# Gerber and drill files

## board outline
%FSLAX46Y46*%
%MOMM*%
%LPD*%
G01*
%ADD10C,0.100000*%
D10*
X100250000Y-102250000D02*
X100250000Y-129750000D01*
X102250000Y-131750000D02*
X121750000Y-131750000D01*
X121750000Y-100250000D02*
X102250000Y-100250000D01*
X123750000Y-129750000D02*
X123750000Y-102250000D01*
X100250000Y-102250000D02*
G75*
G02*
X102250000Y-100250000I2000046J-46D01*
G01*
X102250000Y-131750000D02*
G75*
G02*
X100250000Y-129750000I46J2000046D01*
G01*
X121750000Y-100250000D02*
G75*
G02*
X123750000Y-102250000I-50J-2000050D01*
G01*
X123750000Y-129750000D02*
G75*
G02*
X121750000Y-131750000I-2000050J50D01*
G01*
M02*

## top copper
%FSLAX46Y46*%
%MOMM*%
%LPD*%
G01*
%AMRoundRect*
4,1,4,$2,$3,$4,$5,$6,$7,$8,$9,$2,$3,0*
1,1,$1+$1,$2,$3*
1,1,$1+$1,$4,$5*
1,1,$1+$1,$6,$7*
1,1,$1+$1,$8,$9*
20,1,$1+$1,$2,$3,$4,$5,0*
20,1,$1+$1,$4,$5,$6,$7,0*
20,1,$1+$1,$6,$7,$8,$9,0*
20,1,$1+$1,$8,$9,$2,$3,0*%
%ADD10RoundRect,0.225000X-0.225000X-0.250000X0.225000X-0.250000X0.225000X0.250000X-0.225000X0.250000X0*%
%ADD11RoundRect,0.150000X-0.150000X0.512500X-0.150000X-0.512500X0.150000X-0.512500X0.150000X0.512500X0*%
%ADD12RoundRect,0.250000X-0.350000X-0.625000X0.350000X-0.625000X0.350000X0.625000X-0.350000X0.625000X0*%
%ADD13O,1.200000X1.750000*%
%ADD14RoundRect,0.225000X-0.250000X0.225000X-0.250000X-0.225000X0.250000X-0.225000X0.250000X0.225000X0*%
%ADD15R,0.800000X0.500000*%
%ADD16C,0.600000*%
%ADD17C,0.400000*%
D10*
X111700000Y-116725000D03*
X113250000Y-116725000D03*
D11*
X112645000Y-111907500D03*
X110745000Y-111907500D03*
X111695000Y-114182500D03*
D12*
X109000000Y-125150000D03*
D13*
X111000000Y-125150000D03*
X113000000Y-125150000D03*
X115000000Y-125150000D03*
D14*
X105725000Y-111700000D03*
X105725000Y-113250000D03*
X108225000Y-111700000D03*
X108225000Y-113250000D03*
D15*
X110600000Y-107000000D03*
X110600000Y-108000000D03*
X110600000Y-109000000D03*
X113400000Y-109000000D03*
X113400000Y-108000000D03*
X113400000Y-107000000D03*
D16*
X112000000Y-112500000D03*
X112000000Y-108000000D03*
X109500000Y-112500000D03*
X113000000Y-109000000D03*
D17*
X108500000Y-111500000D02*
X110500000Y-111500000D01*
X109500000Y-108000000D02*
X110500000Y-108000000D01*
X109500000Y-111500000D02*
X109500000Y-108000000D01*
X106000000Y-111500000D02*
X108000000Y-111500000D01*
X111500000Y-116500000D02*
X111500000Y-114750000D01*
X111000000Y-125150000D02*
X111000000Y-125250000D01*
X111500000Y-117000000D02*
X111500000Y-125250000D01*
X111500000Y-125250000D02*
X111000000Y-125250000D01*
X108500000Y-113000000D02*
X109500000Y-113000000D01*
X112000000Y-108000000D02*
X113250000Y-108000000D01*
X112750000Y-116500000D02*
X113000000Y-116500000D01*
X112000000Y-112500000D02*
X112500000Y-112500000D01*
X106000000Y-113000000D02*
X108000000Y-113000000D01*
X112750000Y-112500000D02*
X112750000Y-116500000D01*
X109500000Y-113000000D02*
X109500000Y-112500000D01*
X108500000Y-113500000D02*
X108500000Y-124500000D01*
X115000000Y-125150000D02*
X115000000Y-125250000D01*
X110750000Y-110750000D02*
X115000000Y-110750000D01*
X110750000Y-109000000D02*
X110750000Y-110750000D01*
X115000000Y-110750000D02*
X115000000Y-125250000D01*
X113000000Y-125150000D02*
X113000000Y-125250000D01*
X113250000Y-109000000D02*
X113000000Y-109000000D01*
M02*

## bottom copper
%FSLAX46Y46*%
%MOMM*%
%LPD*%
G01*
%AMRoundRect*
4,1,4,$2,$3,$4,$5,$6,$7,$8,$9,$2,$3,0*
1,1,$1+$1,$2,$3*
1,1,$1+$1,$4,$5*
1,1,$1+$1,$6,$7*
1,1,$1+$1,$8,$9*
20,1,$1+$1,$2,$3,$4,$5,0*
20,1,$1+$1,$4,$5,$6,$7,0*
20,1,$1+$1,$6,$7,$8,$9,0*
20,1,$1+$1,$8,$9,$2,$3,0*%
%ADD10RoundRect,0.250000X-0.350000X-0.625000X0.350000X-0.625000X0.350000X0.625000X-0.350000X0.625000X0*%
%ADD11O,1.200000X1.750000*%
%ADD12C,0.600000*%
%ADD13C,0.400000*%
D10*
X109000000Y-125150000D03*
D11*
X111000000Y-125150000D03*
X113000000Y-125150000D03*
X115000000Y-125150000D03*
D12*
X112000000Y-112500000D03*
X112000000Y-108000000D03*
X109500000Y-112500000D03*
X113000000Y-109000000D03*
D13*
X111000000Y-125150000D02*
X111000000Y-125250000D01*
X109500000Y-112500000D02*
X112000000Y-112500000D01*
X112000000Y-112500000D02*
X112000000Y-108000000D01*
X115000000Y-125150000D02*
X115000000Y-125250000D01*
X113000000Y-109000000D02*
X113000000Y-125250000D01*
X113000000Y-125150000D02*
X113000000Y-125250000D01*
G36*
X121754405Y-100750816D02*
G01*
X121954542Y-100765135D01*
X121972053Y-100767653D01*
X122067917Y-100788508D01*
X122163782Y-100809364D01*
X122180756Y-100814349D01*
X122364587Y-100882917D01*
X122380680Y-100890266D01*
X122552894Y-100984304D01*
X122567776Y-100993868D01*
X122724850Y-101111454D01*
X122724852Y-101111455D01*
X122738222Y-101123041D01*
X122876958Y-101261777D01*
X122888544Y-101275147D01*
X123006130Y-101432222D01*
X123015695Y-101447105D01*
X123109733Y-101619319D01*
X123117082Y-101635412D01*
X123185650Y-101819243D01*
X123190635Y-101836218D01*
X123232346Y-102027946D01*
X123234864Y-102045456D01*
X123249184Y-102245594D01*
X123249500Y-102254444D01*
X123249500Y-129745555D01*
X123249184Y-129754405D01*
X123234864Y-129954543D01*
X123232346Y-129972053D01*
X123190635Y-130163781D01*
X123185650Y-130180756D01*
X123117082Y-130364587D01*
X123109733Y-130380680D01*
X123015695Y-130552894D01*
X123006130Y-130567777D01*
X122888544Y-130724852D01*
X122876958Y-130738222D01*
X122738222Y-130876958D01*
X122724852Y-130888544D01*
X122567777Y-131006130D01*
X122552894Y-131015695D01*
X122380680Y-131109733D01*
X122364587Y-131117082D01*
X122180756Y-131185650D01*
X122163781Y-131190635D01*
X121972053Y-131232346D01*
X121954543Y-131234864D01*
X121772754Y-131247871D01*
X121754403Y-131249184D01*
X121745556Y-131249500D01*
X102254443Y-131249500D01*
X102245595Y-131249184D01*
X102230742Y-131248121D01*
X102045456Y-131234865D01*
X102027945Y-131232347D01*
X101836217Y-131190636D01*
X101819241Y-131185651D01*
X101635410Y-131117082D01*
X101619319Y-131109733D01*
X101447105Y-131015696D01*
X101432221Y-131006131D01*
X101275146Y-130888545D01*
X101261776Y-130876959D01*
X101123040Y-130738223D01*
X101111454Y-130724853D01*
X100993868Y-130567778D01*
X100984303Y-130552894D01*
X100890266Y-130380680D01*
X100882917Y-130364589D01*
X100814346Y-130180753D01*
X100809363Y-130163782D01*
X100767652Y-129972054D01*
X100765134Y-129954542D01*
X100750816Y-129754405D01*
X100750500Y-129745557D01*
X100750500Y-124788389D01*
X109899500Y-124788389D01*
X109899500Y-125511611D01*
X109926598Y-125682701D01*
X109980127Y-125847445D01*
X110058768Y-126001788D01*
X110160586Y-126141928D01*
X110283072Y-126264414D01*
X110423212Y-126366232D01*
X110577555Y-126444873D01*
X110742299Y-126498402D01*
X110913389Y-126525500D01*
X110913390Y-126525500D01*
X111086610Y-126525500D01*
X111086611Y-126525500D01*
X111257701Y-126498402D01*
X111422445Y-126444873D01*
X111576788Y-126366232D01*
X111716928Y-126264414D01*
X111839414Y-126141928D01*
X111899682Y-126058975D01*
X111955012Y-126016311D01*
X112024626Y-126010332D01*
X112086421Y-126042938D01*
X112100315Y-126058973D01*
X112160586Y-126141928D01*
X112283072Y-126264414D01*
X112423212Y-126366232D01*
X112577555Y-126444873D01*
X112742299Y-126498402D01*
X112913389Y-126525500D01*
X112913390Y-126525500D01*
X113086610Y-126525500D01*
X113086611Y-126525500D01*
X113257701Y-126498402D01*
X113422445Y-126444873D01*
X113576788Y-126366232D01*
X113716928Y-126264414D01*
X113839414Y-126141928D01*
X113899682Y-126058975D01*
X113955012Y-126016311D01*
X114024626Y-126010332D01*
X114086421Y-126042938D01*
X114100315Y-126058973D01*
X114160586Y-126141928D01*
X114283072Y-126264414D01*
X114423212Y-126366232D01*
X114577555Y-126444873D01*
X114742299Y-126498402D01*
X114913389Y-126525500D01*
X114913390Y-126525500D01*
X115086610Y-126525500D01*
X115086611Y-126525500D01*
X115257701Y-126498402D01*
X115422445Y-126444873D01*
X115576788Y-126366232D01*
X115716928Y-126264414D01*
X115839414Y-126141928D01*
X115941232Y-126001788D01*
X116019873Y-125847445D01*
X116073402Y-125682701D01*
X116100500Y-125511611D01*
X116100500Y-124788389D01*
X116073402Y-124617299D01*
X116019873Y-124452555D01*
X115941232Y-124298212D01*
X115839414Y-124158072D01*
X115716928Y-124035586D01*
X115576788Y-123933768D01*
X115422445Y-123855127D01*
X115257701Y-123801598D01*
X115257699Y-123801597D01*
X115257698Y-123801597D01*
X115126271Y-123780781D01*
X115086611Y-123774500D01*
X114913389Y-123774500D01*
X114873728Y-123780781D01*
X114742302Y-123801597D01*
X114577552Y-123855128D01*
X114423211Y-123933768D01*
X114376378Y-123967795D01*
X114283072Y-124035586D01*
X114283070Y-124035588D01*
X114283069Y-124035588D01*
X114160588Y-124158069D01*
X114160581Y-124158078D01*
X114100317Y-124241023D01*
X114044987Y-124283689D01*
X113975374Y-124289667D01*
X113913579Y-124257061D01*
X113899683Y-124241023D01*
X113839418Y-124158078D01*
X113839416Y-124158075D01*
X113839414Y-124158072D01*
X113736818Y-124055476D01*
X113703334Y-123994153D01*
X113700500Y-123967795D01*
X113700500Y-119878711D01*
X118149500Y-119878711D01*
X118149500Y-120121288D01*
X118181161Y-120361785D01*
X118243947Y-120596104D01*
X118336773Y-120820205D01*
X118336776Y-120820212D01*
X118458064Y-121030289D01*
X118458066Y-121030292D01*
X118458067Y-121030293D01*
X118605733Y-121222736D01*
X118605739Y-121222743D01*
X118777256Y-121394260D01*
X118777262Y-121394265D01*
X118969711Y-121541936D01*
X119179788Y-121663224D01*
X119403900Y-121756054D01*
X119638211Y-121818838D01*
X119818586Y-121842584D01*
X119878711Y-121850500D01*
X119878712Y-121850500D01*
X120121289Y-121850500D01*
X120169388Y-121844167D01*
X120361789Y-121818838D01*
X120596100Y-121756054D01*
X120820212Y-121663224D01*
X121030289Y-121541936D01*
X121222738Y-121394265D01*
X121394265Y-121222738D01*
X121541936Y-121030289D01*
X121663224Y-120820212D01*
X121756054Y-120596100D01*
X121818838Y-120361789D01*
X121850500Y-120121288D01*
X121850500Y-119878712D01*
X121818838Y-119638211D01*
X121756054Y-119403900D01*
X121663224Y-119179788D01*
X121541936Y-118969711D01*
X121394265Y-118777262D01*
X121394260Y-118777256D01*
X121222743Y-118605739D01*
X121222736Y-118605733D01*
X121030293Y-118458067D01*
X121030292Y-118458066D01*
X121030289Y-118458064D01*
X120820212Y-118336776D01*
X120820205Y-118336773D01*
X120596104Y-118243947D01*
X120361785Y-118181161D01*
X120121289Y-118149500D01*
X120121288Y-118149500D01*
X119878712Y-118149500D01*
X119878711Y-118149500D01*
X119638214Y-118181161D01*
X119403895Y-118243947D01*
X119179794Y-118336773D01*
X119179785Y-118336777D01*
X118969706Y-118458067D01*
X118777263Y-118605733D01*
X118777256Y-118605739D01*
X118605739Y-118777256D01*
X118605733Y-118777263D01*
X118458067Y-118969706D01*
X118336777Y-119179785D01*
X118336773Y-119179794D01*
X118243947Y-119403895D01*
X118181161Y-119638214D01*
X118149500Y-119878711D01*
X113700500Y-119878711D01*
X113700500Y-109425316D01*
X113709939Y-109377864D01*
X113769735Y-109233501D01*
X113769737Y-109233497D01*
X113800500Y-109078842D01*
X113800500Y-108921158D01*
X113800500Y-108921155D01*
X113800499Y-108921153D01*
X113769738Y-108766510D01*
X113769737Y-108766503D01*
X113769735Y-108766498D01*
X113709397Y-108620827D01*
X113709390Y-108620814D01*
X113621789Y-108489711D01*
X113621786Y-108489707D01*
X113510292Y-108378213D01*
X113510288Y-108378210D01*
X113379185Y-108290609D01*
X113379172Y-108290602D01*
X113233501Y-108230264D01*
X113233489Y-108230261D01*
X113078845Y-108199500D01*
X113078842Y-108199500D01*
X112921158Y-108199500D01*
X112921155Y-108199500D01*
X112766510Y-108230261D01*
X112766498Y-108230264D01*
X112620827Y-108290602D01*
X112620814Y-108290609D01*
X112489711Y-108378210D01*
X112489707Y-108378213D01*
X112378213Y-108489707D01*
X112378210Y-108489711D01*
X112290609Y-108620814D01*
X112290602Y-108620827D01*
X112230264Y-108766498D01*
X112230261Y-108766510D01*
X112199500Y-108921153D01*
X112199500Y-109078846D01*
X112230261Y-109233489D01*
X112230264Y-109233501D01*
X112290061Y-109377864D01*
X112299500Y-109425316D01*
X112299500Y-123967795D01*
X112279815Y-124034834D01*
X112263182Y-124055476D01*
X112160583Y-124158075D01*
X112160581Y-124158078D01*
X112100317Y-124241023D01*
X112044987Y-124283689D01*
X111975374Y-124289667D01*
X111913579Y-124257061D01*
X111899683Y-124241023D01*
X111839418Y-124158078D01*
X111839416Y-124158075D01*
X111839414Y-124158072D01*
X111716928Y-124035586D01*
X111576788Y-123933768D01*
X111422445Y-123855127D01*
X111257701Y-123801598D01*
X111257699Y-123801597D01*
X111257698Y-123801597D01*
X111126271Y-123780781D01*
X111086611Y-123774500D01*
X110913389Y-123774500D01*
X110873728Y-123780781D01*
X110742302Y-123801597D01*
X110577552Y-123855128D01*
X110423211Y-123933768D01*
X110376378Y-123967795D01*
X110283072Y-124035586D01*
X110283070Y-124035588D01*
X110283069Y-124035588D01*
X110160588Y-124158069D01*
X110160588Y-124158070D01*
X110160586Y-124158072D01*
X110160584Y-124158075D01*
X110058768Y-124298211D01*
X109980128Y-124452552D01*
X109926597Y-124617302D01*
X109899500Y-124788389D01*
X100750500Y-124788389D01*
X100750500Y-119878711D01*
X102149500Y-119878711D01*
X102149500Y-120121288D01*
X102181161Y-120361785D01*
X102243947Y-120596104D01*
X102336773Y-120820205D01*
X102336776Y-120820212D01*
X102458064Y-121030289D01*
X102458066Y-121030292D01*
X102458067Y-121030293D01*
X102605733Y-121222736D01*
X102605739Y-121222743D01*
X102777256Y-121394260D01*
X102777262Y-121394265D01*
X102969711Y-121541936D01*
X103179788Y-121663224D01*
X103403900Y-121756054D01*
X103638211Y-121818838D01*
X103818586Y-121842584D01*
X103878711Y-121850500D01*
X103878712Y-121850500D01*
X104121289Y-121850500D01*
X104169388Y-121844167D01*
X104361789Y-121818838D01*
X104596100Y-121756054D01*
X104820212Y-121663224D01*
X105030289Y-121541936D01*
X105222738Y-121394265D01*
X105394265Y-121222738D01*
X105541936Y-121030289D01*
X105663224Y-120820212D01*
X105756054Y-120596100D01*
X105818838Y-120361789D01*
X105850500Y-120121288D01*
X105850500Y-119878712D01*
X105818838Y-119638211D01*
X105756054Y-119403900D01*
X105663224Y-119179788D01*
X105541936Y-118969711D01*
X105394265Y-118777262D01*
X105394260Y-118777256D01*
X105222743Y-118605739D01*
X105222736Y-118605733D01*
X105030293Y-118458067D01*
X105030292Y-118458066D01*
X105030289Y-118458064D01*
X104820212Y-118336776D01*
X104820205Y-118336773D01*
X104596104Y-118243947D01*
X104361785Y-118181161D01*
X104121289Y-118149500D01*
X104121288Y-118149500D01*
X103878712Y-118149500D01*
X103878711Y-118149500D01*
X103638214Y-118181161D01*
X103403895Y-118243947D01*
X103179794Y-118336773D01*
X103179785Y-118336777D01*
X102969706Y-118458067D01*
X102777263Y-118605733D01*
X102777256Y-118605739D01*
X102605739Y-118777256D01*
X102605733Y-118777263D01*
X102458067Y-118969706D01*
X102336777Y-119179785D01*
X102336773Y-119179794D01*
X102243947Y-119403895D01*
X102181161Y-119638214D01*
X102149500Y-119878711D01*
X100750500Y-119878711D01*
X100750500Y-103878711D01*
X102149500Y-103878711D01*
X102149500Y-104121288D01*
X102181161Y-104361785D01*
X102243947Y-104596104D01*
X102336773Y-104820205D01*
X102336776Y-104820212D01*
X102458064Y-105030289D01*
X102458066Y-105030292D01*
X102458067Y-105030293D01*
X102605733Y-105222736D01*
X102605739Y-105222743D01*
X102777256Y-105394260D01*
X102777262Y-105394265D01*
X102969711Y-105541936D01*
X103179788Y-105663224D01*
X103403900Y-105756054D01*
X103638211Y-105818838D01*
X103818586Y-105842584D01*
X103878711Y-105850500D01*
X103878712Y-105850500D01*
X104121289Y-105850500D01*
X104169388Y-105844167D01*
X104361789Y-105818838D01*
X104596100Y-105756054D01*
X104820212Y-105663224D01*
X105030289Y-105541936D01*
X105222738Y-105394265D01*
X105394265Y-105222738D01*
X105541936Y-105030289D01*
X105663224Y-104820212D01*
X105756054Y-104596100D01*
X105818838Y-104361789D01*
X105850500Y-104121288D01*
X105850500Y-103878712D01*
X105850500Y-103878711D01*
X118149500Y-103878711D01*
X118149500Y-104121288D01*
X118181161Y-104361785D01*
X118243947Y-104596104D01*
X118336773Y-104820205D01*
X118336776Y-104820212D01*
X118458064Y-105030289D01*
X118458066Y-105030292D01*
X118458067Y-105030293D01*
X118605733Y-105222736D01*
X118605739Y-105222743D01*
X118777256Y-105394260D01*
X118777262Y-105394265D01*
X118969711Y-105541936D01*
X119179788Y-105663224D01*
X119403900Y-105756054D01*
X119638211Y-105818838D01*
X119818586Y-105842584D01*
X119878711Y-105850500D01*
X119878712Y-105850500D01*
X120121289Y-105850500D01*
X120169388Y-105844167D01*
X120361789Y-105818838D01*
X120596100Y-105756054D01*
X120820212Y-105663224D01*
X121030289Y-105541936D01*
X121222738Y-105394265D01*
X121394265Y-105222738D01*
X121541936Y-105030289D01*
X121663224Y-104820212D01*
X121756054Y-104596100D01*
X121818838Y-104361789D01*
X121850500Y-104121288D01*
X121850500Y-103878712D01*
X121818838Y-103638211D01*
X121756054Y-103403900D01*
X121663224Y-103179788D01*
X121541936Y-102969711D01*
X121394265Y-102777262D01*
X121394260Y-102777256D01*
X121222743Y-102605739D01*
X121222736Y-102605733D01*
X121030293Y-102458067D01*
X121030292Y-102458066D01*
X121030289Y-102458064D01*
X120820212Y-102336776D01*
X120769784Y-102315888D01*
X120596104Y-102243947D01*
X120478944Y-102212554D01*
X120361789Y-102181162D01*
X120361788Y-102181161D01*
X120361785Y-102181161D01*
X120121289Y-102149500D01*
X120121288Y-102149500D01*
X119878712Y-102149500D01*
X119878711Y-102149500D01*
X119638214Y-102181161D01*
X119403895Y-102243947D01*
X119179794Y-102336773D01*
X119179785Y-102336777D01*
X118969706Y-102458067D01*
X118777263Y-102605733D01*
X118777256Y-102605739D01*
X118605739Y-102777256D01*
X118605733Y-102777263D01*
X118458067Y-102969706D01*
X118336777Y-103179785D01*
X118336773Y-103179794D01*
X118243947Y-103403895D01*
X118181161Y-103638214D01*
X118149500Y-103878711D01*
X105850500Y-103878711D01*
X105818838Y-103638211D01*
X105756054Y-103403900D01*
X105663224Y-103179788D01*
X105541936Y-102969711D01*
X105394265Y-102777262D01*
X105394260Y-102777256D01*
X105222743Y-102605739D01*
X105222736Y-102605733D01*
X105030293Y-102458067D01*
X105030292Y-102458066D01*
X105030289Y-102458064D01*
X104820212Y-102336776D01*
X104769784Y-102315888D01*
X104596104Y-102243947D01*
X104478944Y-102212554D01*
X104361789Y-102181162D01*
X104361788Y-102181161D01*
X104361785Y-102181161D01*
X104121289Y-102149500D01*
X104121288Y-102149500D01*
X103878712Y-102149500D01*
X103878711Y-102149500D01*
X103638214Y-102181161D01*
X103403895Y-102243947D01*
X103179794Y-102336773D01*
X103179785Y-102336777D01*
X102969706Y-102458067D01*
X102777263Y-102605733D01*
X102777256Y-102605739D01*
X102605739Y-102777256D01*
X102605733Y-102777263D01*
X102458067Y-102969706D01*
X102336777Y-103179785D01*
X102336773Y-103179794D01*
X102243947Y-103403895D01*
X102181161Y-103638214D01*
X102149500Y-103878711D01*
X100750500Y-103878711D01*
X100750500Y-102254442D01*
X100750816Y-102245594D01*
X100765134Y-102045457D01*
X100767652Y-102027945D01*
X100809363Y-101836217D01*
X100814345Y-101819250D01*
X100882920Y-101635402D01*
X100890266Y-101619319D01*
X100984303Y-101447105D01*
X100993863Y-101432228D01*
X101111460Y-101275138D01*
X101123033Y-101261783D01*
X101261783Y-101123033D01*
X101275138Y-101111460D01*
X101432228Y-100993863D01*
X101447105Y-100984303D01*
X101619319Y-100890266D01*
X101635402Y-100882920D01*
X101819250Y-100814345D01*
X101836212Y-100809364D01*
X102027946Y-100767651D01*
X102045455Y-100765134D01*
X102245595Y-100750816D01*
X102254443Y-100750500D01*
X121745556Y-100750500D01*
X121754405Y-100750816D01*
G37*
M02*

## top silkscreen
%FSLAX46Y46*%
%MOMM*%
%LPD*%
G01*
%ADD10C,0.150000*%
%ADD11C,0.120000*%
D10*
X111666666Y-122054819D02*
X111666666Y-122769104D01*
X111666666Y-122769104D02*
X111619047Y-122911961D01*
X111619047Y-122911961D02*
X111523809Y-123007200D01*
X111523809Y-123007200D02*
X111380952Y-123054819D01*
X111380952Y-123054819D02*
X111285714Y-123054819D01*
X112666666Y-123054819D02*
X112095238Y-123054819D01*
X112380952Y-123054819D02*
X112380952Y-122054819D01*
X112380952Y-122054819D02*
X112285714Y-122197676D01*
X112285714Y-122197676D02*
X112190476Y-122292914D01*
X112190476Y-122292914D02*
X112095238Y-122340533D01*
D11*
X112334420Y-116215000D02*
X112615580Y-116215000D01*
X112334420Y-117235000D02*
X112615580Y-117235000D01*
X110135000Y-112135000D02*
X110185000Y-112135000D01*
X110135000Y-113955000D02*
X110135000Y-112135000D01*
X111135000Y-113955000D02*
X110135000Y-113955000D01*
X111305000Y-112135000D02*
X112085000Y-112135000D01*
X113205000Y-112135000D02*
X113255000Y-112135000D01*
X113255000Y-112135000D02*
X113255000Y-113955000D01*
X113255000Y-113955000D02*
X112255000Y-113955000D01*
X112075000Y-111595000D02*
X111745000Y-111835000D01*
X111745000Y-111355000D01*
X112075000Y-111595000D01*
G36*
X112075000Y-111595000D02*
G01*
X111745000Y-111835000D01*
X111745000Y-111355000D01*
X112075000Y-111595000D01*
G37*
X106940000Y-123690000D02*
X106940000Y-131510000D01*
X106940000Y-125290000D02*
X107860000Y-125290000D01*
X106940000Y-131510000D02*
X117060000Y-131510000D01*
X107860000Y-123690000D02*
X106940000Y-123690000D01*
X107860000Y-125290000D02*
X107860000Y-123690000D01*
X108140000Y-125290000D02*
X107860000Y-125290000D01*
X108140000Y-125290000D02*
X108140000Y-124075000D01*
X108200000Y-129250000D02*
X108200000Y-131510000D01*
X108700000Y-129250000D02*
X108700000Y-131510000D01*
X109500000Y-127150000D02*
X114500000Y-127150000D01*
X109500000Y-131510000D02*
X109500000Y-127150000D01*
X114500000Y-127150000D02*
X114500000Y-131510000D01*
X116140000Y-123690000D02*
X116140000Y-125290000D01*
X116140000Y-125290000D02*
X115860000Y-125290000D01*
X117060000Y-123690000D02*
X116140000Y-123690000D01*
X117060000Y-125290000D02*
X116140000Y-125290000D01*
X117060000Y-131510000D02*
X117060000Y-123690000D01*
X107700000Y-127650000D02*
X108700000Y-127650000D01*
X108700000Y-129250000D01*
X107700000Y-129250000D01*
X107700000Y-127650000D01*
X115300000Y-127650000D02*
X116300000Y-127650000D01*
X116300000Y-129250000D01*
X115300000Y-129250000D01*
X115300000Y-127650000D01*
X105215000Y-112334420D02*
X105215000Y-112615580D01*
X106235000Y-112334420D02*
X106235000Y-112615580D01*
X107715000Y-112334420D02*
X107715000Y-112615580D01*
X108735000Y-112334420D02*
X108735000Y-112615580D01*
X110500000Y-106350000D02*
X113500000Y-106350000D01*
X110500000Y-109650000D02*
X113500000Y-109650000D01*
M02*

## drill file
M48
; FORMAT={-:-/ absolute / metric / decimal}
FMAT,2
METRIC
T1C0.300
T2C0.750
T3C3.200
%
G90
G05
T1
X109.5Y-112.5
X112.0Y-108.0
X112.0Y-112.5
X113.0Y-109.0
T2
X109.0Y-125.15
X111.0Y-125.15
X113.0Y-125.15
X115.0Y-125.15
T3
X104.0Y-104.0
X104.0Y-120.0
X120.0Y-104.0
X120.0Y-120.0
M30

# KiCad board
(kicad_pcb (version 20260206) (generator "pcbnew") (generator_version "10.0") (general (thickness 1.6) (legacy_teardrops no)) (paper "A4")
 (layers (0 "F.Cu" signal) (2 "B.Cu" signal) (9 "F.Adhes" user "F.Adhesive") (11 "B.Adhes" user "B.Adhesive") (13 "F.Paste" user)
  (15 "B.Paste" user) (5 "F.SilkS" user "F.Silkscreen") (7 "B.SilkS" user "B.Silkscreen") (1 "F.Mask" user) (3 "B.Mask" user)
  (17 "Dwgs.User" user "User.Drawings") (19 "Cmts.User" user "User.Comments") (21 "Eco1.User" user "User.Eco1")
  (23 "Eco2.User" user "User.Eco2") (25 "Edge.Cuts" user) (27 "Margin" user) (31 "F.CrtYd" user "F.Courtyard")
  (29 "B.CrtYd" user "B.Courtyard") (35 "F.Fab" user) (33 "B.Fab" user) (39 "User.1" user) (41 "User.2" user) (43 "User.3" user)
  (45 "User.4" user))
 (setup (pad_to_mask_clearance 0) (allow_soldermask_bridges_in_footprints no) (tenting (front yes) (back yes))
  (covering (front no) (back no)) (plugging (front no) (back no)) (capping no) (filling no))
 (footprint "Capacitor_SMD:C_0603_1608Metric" (layer "F.Cu") (at 112.475 116.725)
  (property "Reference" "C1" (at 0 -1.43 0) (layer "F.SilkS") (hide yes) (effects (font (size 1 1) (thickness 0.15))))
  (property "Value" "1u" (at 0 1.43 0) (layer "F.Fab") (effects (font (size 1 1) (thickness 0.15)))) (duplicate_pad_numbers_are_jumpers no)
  (fp_line (start -0.14058 -0.51) (end 0.14058 -0.51) (stroke (width 0.12) (type solid)) (layer "F.SilkS"))
  (fp_line (start -0.14058 0.51) (end 0.14058 0.51) (stroke (width 0.12) (type solid)) (layer "F.SilkS"))
  (pad "1" smd roundrect (at -0.775 0) (size 0.9 0.95) (layers "F.Cu" "F.Mask" "F.Paste") (roundrect_rratio 0.25) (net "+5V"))
  (pad "2" smd roundrect (at 0.775 0) (size 0.9 0.95) (layers "F.Cu" "F.Mask" "F.Paste") (roundrect_rratio 0.25) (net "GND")))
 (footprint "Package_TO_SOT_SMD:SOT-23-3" (layer "F.Cu") (at 111.695 113.045 -90)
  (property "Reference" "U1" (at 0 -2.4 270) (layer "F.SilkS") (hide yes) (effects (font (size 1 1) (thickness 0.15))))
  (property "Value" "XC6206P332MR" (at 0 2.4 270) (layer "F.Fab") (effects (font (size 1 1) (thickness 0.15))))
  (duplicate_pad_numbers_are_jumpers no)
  (fp_line (start -0.91 1.56) (end -0.91 1.51) (stroke (width 0.12) (type solid)) (layer "F.SilkS"))
  (fp_line (start 0.91 1.56) (end -0.91 1.56) (stroke (width 0.12) (type solid)) (layer "F.SilkS"))
  (fp_line (start 0.91 0.56) (end 0.91 1.56) (stroke (width 0.12) (type solid)) (layer "F.SilkS"))
  (fp_line (start -0.91 0.39) (end -0.91 -0.39) (stroke (width 0.12) (type solid)) (layer "F.SilkS"))
  (fp_line (start -0.91 -1.51) (end -0.91 -1.56) (stroke (width 0.12) (type solid)) (layer "F.SilkS"))
  (fp_line (start -0.91 -1.56) (end 0.91 -1.56) (stroke (width 0.12) (type solid)) (layer "F.SilkS"))
  (fp_line (start 0.91 -1.56) (end 0.91 -0.56) (stroke (width 0.12) (type solid)) (layer "F.SilkS"))
  (fp_poly (pts (xy -1.45 -0.38) (xy -1.21 -0.05) (xy -1.69 -0.05)) (stroke (width 0.12) (type solid)) (fill yes) (layer "F.SilkS"))
  (pad "1" smd roundrect (at -1.1375 -0.95 270) (size 1.325 0.6) (layers "F.Cu" "F.Mask" "F.Paste") (roundrect_rratio 0.25) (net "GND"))
  (pad "2" smd roundrect (at -1.1375 0.95 270) (size 1.325 0.6) (layers "F.Cu" "F.Mask" "F.Paste") (roundrect_rratio 0.25) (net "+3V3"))
  (pad "3" smd roundrect (at 1.1375 0 270) (size 1.325 0.6) (layers "F.Cu" "F.Mask" "F.Paste") (roundrect_rratio 0.25) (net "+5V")))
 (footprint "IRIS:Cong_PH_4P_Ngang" (layer "F.Cu") (at 109 125.15)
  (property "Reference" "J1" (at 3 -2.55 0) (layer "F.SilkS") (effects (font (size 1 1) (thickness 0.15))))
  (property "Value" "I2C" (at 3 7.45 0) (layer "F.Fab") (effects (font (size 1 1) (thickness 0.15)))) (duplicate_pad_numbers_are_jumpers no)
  (fp_line (start -2.06 -1.46) (end -2.06 6.36) (stroke (width 0.12) (type solid)) (layer "F.SilkS"))
  (fp_line (start -2.06 0.14) (end -1.14 0.14) (stroke (width 0.12) (type solid)) (layer "F.SilkS"))
  (fp_line (start -2.06 6.36) (end 8.06 6.36) (stroke (width 0.12) (type solid)) (layer "F.SilkS"))
  (fp_line (start -1.14 -1.46) (end -2.06 -1.46) (stroke (width 0.12) (type solid)) (layer "F.SilkS"))
  (fp_line (start -1.14 0.14) (end -1.14 -1.46) (stroke (width 0.12) (type solid)) (layer "F.SilkS"))
  (fp_line (start -0.86 0.14) (end -1.14 0.14) (stroke (width 0.12) (type solid)) (layer "F.SilkS"))
  (fp_line (start -0.86 0.14) (end -0.86 -1.075) (stroke (width 0.12) (type solid)) (layer "F.SilkS"))
  (fp_line (start -0.8 4.1) (end -0.8 6.36) (stroke (width 0.12) (type solid)) (layer "F.SilkS"))
  (fp_line (start -0.3 4.1) (end -0.3 6.36) (stroke (width 0.12) (type solid)) (layer "F.SilkS"))
  (fp_line (start 0.5 2) (end 5.5 2) (stroke (width 0.12) (type solid)) (layer "F.SilkS"))
  (fp_line (start 0.5 6.36) (end 0.5 2) (stroke (width 0.12) (type solid)) (layer "F.SilkS"))
  (fp_line (start 5.5 2) (end 5.5 6.36) (stroke (width 0.12) (type solid)) (layer "F.SilkS"))
  (fp_line (start 7.14 -1.46) (end 7.14 0.14) (stroke (width 0.12) (type solid)) (layer "F.SilkS"))
  (fp_line (start 7.14 0.14) (end 6.86 0.14) (stroke (width 0.12) (type solid)) (layer "F.SilkS"))
  (fp_line (start 8.06 -1.46) (end 7.14 -1.46) (stroke (width 0.12) (type solid)) (layer "F.SilkS"))
  (fp_line (start 8.06 0.14) (end 7.14 0.14) (stroke (width 0.12) (type solid)) (layer "F.SilkS"))
  (fp_line (start 8.06 6.36) (end 8.06 -1.46) (stroke (width 0.12) (type solid)) (layer "F.SilkS"))
  (fp_rect (start -1.3 2.5) (end -0.3 4.1) (stroke (width 0.12) (type solid)) (fill no) (layer "F.SilkS"))
  (fp_rect (start 6.3 2.5) (end 7.3 4.1) (stroke (width 0.12) (type solid)) (fill no) (layer "F.SilkS"))
  (pad "1" thru_hole roundrect (at 0 0) (size 1.2 1.75) (drill 0.75) (layers "*.Cu" "*.Mask") (remove_unused_layers no)
   (roundrect_rratio 0.208333) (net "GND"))
  (pad "2" thru_hole oval (at 2 0) (size 1.2 1.75) (drill 0.75) (layers "*.Cu" "*.Mask") (remove_unused_layers no) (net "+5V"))
  (pad "3" thru_hole oval (at 4 0) (size 1.2 1.75) (drill 0.75) (layers "*.Cu" "*.Mask") (remove_unused_layers no) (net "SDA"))
  (pad "4" thru_hole oval (at 6 0) (size 1.2 1.75) (drill 0.75) (layers "*.Cu" "*.Mask") (remove_unused_layers no) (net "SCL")))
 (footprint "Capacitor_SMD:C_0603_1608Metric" (layer "F.Cu") (at 105.725 112.475 -90)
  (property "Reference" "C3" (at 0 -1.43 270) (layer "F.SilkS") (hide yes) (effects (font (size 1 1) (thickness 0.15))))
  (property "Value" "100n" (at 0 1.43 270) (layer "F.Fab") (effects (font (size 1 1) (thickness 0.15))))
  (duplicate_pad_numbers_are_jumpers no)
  (fp_line (start -0.14058 0.51) (end 0.14058 0.51) (stroke (width 0.12) (type solid)) (layer "F.SilkS"))
  (fp_line (start -0.14058 -0.51) (end 0.14058 -0.51) (stroke (width 0.12) (type solid)) (layer "F.SilkS"))
  (pad "1" smd roundrect (at -0.775 0 270) (size 0.9 0.95) (layers "F.Cu" "F.Mask" "F.Paste") (roundrect_rratio 0.25) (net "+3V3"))
  (pad "2" smd roundrect (at 0.775 0 270) (size 0.9 0.95) (layers "F.Cu" "F.Mask" "F.Paste") (roundrect_rratio 0.25) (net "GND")))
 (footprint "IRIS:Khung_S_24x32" (layer "F.Cu") (at 100 132)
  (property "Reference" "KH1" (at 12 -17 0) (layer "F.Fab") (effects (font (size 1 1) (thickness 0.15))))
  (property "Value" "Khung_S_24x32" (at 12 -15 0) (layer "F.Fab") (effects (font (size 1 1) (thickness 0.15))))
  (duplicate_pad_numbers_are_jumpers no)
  (fp_line (start 0.25 -29.75) (end 0.25 -2.25) (stroke (width 0.1) (type solid)) (layer "Edge.Cuts"))
  (fp_line (start 2.25 -0.25) (end 21.75 -0.25) (stroke (width 0.1) (type solid)) (layer "Edge.Cuts"))
  (fp_line (start 21.75 -31.75) (end 2.25 -31.75) (stroke (width 0.1) (type solid)) (layer "Edge.Cuts"))
  (fp_line (start 23.75 -2.25) (end 23.75 -29.75) (stroke (width 0.1) (type solid)) (layer "Edge.Cuts"))
  (fp_arc (start 0.25 -29.75) (mid 0.8358 -31.1642) (end 2.25 -31.75) (stroke (width 0.1) (type solid)) (layer "Edge.Cuts"))
  (fp_arc (start 2.25 -0.25) (mid 0.8358 -0.8358) (end 0.25 -2.25) (stroke (width 0.1) (type solid)) (layer "Edge.Cuts"))
  (fp_arc (start 21.75 -31.75) (mid 23.164199 -31.164199) (end 23.75 -29.75) (stroke (width 0.1) (type solid)) (layer "Edge.Cuts"))
  (fp_arc (start 23.75 -2.25) (mid 23.164199 -0.835801) (end 21.75 -0.25) (stroke (width 0.1) (type solid)) (layer "Edge.Cuts"))
  (pad "" np_thru_hole circle (at 4 -28) (size 3.2 3.2) (drill 3.2) (layers "*.Cu" "*.Mask"))
  (pad "" np_thru_hole circle (at 4 -12) (size 3.2 3.2) (drill 3.2) (layers "*.Cu" "*.Mask"))
  (pad "" np_thru_hole circle (at 20 -28) (size 3.2 3.2) (drill 3.2) (layers "*.Cu" "*.Mask"))
  (pad "" np_thru_hole circle (at 20 -12) (size 3.2 3.2) (drill 3.2) (layers "*.Cu" "*.Mask")))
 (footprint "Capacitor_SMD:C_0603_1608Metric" (layer "F.Cu") (at 108.225 112.475 -90)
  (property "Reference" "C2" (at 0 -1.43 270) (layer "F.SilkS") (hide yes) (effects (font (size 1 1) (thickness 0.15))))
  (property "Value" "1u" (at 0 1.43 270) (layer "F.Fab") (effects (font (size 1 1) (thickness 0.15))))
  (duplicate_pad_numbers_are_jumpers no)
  (fp_line (start -0.14058 0.51) (end 0.14058 0.51) (stroke (width 0.12) (type solid)) (layer "F.SilkS"))
  (fp_line (start -0.14058 -0.51) (end 0.14058 -0.51) (stroke (width 0.12) (type solid)) (layer "F.SilkS"))
  (pad "1" smd roundrect (at -0.775 0 270) (size 0.9 0.95) (layers "F.Cu" "F.Mask" "F.Paste") (roundrect_rratio 0.25) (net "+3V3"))
  (pad "2" smd roundrect (at 0.775 0 270) (size 0.9 0.95) (layers "F.Cu" "F.Mask" "F.Paste") (roundrect_rratio 0.25) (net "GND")))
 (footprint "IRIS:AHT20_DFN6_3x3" (layer "F.Cu") (at 112 108)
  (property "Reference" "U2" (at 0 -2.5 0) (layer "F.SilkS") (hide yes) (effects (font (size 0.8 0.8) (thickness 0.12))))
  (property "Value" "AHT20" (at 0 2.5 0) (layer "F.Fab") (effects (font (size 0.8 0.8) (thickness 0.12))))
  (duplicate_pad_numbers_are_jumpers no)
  (fp_line (start -1.5 -1.65) (end 1.5 -1.65) (stroke (width 0.12) (type solid)) (layer "F.SilkS"))
  (fp_line (start -1.5 1.65) (end 1.5 1.65) (stroke (width 0.12) (type solid)) (layer "F.SilkS"))
  (pad "1" smd rect (at -1.4 -1) (size 0.8 0.5) (layers "F.Cu" "F.Mask" "F.Paste") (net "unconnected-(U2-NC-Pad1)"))
  (pad "2" smd rect (at -1.4 0) (size 0.8 0.5) (layers "F.Cu" "F.Mask" "F.Paste") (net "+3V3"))
  (pad "3" smd rect (at -1.4 1) (size 0.8 0.5) (layers "F.Cu" "F.Mask" "F.Paste") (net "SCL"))
  (pad "4" smd rect (at 1.4 1) (size 0.8 0.5) (layers "F.Cu" "F.Mask" "F.Paste") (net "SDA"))
  (pad "5" smd rect (at 1.4 0) (size 0.8 0.5) (layers "F.Cu" "F.Mask" "F.Paste") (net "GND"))
  (pad "6" smd rect (at 1.4 -1) (size 0.8 0.5) (layers "F.Cu" "F.Mask" "F.Paste") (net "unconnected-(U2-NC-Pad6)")))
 (segment (start 108.5 111.5) (end 110.5 111.5) (width 0.4) (layer "F.Cu") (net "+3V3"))
 (segment (start 109.5 108) (end 110.5 108) (width 0.4) (layer "F.Cu") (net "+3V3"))
 (segment (start 109.5 111.5) (end 109.5 108) (width 0.4) (layer "F.Cu") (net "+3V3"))
 (segment (start 106 111.5) (end 108 111.5) (width 0.4) (layer "F.Cu") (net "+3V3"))
 (segment (start 111.5 116.5) (end 111.5 114.75) (width 0.4) (layer "F.Cu") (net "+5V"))
 (segment (start 111 125.15) (end 111 125.25) (width 0.4) (layer "F.Cu") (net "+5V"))
 (segment (start 111.5 117) (end 111.5 125.25) (width 0.4) (layer "F.Cu") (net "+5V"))
 (segment (start 111.5 125.25) (end 111 125.25) (width 0.4) (layer "F.Cu") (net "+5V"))
 (segment (start 111 125.15) (end 111 125.25) (width 0.4) (layer "B.Cu") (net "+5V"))
 (segment (start 108.5 113) (end 109.5 113) (width 0.4) (layer "F.Cu") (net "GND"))
 (segment (start 112 108) (end 113.25 108) (width 0.4) (layer "F.Cu") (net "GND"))
 (segment (start 112.75 116.5) (end 113 116.5) (width 0.4) (layer "F.Cu") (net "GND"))
 (segment (start 112 112.5) (end 112.5 112.5) (width 0.4) (layer "F.Cu") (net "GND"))
 (segment (start 106 113) (end 108 113) (width 0.4) (layer "F.Cu") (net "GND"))
 (segment (start 112.75 112.5) (end 112.75 116.5) (width 0.4) (layer "F.Cu") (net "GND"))
 (segment (start 109.5 113) (end 109.5 112.5) (width 0.4) (layer "F.Cu") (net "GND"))
 (segment (start 108.5 113.5) (end 108.5 124.5) (width 0.4) (layer "F.Cu") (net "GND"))
 (via (at 112 112.5) (size 0.6) (drill 0.3) (layers "F.Cu" "B.Cu") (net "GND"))
 (via (at 112 108) (size 0.6) (drill 0.3) (layers "F.Cu" "B.Cu") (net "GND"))
 (via (at 109.5 112.5) (size 0.6) (drill 0.3) (layers "F.Cu" "B.Cu") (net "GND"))
 (segment (start 109.5 112.5) (end 112 112.5) (width 0.4) (layer "B.Cu") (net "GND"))
 (segment (start 112 112.5) (end 112 108) (width 0.4) (layer "B.Cu") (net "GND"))
 (segment (start 115 125.15) (end 115 125.25) (width 0.4) (layer "F.Cu") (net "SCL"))
 (segment (start 110.75 110.75) (end 115 110.75) (width 0.4) (layer "F.Cu") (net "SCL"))
 (segment (start 110.75 109) (end 110.75 110.75) (width 0.4) (layer "F.Cu") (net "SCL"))
 (segment (start 115 110.75) (end 115 125.25) (width 0.4) (layer "F.Cu") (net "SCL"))
 (segment (start 115 125.15) (end 115 125.25) (width 0.4) (layer "B.Cu") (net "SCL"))
 (segment (start 113 125.15) (end 113 125.25) (width 0.4) (layer "F.Cu") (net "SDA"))
 (segment (start 113.25 109) (end 113 109) (width 0.4) (layer "F.Cu") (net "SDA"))
 (via (at 113 109) (size 0.6) (drill 0.3) (layers "F.Cu" "B.Cu") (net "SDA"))
 (segment (start 113 109) (end 113 125.25) (width 0.4) (layer "B.Cu") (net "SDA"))
 (segment (start 113 125.15) (end 113 125.25) (width 0.4) (layer "B.Cu") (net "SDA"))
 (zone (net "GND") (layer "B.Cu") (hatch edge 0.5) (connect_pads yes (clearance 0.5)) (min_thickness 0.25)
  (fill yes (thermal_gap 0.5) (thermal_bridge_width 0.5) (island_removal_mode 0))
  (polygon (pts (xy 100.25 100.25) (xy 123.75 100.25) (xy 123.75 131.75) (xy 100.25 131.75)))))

